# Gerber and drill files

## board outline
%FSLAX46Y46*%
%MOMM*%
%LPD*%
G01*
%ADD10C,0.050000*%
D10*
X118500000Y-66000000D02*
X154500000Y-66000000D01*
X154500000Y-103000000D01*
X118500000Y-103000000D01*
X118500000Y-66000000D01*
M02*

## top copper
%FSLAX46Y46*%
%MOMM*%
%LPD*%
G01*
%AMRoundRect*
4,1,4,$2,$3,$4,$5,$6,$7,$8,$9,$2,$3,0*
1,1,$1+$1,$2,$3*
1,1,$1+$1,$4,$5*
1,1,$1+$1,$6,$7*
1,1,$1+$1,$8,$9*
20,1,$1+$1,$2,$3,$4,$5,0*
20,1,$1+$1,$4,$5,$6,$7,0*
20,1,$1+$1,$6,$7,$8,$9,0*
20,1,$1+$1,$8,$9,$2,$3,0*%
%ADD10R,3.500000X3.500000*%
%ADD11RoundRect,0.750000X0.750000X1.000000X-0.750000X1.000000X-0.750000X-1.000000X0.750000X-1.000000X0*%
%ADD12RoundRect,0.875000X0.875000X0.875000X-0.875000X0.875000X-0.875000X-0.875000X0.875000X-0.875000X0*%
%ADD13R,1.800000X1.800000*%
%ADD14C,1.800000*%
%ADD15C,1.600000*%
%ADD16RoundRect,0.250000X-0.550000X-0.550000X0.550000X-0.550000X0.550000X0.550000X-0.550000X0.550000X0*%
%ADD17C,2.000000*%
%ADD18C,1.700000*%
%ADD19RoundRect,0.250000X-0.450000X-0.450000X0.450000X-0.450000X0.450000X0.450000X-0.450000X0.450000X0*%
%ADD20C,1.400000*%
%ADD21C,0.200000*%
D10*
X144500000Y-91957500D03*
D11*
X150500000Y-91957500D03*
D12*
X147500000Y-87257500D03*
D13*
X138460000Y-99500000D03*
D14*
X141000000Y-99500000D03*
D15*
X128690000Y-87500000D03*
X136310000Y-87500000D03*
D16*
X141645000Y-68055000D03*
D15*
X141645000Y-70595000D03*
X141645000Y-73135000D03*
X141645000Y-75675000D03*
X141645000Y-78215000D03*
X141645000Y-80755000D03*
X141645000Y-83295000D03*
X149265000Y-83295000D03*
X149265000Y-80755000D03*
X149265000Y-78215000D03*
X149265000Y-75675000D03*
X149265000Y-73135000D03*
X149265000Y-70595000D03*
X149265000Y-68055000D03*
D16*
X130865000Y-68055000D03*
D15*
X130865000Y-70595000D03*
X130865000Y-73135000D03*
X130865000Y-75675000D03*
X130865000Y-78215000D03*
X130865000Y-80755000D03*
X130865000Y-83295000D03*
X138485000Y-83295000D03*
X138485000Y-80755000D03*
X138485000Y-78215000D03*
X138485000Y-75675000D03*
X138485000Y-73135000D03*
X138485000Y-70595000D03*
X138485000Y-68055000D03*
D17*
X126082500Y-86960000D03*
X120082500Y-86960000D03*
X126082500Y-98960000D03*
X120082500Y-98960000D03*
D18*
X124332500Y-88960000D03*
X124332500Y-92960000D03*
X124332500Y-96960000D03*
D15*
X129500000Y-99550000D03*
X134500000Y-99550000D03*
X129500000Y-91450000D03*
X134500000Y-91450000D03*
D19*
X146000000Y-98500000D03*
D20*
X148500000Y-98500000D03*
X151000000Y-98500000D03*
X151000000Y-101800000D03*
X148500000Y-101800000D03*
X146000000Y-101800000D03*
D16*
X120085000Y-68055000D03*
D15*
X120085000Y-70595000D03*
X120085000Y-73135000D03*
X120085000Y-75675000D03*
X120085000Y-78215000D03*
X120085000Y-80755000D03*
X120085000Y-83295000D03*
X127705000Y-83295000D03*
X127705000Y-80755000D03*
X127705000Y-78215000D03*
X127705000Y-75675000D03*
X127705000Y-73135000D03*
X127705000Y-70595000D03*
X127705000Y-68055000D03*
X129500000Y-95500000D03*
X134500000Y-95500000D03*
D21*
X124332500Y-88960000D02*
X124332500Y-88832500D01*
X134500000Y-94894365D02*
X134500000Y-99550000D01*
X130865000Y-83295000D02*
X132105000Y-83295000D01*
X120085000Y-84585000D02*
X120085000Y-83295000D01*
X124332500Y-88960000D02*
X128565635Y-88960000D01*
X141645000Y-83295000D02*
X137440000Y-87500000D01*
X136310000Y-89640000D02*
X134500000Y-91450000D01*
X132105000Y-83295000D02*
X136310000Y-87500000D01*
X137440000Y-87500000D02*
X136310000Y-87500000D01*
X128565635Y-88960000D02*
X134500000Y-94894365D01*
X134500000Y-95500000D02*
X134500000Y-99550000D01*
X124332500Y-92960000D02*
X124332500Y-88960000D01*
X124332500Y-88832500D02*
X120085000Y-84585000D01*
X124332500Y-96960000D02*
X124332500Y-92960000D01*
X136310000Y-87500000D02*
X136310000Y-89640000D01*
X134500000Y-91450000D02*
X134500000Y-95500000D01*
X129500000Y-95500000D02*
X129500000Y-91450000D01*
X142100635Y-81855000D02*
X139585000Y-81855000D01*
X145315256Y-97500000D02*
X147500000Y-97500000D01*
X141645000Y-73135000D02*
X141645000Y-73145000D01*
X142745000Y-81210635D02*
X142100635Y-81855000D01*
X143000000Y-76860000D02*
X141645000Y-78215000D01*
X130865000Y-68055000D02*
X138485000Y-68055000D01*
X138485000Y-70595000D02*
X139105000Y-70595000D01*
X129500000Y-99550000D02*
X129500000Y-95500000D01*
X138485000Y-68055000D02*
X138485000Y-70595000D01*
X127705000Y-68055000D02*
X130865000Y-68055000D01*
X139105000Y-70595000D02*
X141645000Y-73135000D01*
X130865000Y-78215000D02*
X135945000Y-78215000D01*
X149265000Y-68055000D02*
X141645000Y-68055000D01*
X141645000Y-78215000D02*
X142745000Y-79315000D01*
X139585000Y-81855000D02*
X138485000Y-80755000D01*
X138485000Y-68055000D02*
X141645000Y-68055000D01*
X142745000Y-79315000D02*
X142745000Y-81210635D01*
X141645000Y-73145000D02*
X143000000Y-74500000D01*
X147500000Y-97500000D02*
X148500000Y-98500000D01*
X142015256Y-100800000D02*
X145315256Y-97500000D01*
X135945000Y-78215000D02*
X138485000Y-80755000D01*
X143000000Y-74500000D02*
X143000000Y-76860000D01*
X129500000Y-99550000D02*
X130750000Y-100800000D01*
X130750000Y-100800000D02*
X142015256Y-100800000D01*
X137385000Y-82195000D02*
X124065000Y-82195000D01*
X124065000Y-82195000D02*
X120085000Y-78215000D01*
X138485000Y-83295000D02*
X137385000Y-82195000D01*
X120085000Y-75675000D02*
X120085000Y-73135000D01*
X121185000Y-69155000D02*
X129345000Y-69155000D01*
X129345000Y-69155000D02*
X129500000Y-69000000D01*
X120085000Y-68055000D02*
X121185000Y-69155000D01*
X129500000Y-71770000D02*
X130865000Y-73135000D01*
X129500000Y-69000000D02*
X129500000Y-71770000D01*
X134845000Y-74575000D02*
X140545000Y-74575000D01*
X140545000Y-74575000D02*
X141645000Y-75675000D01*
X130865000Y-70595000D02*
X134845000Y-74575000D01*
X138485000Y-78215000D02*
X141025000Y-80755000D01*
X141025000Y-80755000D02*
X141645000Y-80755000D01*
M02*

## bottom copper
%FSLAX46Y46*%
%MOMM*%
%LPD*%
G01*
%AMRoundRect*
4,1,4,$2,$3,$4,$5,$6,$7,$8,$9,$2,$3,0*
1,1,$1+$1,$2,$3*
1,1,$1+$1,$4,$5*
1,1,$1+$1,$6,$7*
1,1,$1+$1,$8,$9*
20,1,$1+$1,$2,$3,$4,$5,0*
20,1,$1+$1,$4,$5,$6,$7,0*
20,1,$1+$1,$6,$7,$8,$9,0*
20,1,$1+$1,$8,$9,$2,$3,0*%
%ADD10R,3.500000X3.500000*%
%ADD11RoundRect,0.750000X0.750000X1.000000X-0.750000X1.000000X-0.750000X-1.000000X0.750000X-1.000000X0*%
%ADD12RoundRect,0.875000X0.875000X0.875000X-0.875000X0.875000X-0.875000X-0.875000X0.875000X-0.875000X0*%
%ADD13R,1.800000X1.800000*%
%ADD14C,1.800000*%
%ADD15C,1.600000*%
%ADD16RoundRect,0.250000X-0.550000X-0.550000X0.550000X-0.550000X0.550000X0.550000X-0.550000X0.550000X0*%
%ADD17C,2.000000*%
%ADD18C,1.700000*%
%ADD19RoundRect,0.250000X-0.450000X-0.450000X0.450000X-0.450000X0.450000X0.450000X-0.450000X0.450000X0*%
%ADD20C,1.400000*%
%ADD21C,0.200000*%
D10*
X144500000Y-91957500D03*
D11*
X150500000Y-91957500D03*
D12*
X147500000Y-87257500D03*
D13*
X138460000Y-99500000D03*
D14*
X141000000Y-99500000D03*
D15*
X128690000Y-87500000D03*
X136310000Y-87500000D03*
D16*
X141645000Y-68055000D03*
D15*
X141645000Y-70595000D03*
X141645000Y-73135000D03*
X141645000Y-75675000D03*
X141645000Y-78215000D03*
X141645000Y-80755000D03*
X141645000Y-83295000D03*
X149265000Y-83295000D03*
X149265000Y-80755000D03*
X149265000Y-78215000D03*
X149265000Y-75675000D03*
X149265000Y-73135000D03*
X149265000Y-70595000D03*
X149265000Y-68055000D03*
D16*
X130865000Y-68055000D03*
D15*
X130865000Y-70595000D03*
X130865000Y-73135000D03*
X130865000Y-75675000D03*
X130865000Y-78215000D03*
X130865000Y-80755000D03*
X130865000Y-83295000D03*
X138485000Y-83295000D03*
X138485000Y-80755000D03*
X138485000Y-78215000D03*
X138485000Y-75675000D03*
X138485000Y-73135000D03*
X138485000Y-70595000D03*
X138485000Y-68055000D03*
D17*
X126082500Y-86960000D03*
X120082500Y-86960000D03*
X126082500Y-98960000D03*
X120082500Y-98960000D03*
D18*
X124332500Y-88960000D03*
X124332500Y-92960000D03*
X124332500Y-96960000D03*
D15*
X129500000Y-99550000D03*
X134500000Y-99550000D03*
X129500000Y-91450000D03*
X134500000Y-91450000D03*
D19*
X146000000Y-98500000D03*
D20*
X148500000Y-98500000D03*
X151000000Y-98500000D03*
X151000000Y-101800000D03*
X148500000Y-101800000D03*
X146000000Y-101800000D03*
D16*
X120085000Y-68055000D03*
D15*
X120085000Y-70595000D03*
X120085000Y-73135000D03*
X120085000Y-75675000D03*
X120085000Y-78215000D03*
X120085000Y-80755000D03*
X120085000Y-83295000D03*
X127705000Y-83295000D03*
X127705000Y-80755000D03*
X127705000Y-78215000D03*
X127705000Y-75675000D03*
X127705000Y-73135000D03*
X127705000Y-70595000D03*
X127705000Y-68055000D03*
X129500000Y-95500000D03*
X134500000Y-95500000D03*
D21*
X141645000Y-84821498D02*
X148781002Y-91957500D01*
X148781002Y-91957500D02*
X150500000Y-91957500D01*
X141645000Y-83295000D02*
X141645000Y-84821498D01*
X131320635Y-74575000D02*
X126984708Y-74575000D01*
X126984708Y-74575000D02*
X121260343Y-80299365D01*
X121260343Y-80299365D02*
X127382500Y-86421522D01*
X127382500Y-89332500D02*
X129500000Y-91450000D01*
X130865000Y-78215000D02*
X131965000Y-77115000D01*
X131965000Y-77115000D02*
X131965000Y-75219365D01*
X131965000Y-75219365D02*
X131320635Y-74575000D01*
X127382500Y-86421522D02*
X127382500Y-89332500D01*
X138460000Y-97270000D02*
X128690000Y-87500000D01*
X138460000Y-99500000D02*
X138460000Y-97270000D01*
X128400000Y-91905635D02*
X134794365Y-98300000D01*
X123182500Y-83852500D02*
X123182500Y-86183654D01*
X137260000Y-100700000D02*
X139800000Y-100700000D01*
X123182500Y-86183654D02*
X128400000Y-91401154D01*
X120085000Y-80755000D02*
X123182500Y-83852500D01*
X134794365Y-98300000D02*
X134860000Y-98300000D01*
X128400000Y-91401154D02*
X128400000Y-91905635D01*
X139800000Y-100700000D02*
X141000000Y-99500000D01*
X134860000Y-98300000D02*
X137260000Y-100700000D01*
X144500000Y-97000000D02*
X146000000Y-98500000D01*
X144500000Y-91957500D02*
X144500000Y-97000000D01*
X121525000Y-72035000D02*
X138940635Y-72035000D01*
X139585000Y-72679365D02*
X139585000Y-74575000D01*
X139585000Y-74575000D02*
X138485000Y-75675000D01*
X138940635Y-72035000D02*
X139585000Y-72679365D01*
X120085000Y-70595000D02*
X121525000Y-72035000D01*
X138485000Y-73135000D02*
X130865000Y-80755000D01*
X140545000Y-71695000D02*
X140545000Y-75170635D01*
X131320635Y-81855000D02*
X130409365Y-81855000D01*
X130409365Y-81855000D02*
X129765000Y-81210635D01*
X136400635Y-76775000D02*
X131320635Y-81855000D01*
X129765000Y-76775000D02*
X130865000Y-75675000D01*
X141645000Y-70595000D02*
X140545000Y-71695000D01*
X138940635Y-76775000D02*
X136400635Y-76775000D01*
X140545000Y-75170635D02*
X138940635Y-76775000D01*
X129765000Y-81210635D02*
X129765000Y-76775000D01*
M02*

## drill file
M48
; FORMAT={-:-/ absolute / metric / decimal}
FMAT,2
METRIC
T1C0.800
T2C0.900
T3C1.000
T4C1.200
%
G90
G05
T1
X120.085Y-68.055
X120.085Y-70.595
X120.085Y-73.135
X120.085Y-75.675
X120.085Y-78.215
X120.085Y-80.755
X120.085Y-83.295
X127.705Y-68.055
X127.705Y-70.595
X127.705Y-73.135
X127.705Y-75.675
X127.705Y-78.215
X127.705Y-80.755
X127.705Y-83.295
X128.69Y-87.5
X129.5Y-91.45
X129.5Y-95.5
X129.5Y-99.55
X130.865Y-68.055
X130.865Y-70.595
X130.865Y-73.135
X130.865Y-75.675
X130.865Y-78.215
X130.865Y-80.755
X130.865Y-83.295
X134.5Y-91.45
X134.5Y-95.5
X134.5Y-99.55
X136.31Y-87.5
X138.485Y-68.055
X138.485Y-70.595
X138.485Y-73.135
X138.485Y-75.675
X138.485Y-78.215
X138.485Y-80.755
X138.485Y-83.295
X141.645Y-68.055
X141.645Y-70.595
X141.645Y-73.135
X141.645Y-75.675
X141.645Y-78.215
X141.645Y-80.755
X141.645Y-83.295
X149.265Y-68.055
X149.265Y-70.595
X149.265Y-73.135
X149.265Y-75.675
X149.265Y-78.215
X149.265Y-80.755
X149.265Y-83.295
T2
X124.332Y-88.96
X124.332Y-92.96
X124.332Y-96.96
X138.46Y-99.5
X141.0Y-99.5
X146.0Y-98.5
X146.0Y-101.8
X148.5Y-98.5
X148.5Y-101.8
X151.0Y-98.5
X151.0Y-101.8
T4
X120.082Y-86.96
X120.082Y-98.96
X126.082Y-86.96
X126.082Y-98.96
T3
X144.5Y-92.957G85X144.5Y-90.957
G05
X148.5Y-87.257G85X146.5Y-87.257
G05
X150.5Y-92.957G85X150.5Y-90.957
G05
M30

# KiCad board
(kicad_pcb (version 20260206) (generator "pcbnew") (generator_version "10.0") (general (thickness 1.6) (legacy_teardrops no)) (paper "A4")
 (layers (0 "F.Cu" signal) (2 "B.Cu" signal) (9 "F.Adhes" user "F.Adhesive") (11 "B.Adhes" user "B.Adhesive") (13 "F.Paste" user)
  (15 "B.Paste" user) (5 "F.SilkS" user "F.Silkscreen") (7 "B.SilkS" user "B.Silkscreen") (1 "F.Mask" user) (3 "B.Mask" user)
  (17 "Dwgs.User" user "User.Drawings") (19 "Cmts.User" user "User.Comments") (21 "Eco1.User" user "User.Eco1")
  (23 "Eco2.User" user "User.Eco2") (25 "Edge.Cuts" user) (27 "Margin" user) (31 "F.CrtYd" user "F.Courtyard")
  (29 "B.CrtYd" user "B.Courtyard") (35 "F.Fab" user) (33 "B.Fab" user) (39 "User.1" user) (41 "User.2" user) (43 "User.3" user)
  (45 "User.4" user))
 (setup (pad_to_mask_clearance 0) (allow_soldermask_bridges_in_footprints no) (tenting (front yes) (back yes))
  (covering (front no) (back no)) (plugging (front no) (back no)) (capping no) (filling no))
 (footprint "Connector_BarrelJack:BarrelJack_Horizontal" (layer "F.Cu") (at 144.5 91.9575 180)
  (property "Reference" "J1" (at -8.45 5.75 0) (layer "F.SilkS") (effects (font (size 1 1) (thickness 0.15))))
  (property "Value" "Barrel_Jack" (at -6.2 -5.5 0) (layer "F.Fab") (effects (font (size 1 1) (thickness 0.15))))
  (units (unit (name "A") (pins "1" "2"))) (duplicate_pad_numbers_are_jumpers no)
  (pad "1" thru_hole rect (at 0 0 180) (size 3.5 3.5) (drill oval 1 3) (layers "*.Cu" "*.Mask") (remove_unused_layers no)
   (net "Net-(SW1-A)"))
  (pad "2" thru_hole roundrect (at -6 0 180) (size 3 3.5) (drill oval 1 3) (layers "*.Cu" "*.Mask") (remove_unused_layers no)
   (roundrect_rratio 0.25) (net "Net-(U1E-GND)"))
  (pad "3" thru_hole roundrect (at -3 4.7 180) (size 3.5 3.5) (drill oval 3 1) (layers "*.Cu" "*.Mask") (remove_unused_layers no)
   (roundrect_rratio 0.25)))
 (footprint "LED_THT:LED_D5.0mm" (layer "F.Cu") (at 138.46 99.5)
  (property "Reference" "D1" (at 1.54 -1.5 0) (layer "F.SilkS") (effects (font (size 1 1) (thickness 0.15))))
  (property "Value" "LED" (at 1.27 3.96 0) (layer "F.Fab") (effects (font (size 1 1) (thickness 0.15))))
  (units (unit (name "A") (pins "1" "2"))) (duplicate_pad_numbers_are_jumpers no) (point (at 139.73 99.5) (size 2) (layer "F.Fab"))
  (pad "1" thru_hole rect (at 0 0) (size 1.8 1.8) (drill 0.9) (layers "*.Cu" "*.Mask") (remove_unused_layers no) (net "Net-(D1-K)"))
  (pad "2" thru_hole circle (at 2.54 0) (size 1.8 1.8) (drill 0.9) (layers "*.Cu" "*.Mask") (remove_unused_layers no) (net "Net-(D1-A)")))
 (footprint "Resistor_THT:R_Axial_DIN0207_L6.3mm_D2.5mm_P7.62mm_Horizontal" (layer "F.Cu") (at 128.69 87.5)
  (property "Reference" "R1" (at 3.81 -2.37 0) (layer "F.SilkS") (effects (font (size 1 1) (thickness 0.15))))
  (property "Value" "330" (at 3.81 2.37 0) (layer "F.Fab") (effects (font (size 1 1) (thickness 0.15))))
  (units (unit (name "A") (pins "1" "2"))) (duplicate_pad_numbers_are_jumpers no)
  (pad "1" thru_hole circle (at 0 0) (size 1.6 1.6) (drill 0.8) (layers "*.Cu" "*.Mask") (remove_unused_layers no) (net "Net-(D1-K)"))
  (pad "2" thru_hole circle (at 7.62 0) (size 1.6 1.6) (drill 0.8) (layers "*.Cu" "*.Mask") (remove_unused_layers no) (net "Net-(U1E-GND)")))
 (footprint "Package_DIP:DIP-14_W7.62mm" (layer "F.Cu") (at 141.645 68.055)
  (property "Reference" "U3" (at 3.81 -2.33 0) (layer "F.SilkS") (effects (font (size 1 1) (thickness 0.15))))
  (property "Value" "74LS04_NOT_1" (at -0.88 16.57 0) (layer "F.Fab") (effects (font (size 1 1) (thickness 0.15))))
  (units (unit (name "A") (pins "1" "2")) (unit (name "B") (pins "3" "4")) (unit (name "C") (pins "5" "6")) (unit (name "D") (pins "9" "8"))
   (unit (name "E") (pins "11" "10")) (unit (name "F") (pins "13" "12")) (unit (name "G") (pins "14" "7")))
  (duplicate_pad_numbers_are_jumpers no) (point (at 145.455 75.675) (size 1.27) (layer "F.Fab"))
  (pad "1" thru_hole roundrect (at 0 0) (size 1.6 1.6) (drill 0.8) (layers "*.Cu" "*.Mask") (remove_unused_layers no)
   (roundrect_rratio 0.15625) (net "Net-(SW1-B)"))
  (pad "2" thru_hole circle (at 0 2.54) (size 1.6 1.6) (drill 0.8) (layers "*.Cu" "*.Mask") (remove_unused_layers no) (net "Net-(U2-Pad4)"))
  (pad "3" thru_hole circle (at 0 5.08) (size 1.6 1.6) (drill 0.8) (layers "*.Cu" "*.Mask") (remove_unused_layers no) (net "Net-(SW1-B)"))
  (pad "4" thru_hole circle (at 0 7.62) (size 1.6 1.6) (drill 0.8) (layers "*.Cu" "*.Mask") (remove_unused_layers no) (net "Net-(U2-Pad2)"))
  (pad "5" thru_hole circle (at 0 10.16) (size 1.6 1.6) (drill 0.8) (layers "*.Cu" "*.Mask") (remove_unused_layers no) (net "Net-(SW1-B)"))
  (pad "6" thru_hole circle (at 0 12.7) (size 1.6 1.6) (drill 0.8) (layers "*.Cu" "*.Mask") (remove_unused_layers no) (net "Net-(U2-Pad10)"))
  (pad "7" thru_hole circle (at 0 15.24) (size 1.6 1.6) (drill 0.8) (layers "*.Cu" "*.Mask") (remove_unused_layers no) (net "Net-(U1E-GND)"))
  (pad "8" thru_hole circle (at 7.62 15.24) (size 1.6 1.6) (drill 0.8) (layers "*.Cu" "*.Mask") (remove_unused_layers no)
   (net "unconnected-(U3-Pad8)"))
  (pad "9" thru_hole circle (at 7.62 12.7) (size 1.6 1.6) (drill 0.8) (layers "*.Cu" "*.Mask") (remove_unused_layers no)
   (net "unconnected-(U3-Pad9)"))
  (pad "10" thru_hole circle (at 7.62 10.16) (size 1.6 1.6) (drill 0.8) (layers "*.Cu" "*.Mask") (remove_unused_layers no)
   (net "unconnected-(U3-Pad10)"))
  (pad "11" thru_hole circle (at 7.62 7.62) (size 1.6 1.6) (drill 0.8) (layers "*.Cu" "*.Mask") (remove_unused_layers no)
   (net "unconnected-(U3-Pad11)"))
  (pad "12" thru_hole circle (at 7.62 5.08) (size 1.6 1.6) (drill 0.8) (layers "*.Cu" "*.Mask") (remove_unused_layers no)
   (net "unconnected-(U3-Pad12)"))
  (pad "13" thru_hole circle (at 7.62 2.54) (size 1.6 1.6) (drill 0.8) (layers "*.Cu" "*.Mask") (remove_unused_layers no)
   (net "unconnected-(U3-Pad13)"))
  (pad "14" thru_hole circle (at 7.62 0) (size 1.6 1.6) (drill 0.8) (layers "*.Cu" "*.Mask") (remove_unused_layers no) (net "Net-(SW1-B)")))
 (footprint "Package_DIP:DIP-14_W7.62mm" (layer "F.Cu") (at 130.865 68.055)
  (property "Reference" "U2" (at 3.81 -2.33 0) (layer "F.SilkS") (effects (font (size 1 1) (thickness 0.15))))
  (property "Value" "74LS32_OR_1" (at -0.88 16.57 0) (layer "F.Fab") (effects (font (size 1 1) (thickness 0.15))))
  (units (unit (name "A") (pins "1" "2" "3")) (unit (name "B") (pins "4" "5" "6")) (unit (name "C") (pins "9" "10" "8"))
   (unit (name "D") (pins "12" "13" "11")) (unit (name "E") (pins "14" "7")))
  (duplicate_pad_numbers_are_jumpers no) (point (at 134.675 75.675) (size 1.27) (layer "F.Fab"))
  (pad "1" thru_hole roundrect (at 0 0) (size 1.6 1.6) (drill 0.8) (layers "*.Cu" "*.Mask") (remove_unused_layers no)
   (roundrect_rratio 0.15625) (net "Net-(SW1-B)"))
  (pad "2" thru_hole circle (at 0 2.54) (size 1.6 1.6) (drill 0.8) (layers "*.Cu" "*.Mask") (remove_unused_layers no) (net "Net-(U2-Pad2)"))
  (pad "3" thru_hole circle (at 0 5.08) (size 1.6 1.6) (drill 0.8) (layers "*.Cu" "*.Mask") (remove_unused_layers no) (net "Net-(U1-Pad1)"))
  (pad "4" thru_hole circle (at 0 7.62) (size 1.6 1.6) (drill 0.8) (layers "*.Cu" "*.Mask") (remove_unused_layers no) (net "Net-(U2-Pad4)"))
  (pad "5" thru_hole circle (at 0 10.16) (size 1.6 1.6) (drill 0.8) (layers "*.Cu" "*.Mask") (remove_unused_layers no) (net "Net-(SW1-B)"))
  (pad "6" thru_hole circle (at 0 12.7) (size 1.6 1.6) (drill 0.8) (layers "*.Cu" "*.Mask") (remove_unused_layers no) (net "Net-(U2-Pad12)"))
  (pad "7" thru_hole circle (at 0 15.24) (size 1.6 1.6) (drill 0.8) (layers "*.Cu" "*.Mask") (remove_unused_layers no) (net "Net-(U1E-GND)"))
  (pad "8" thru_hole circle (at 7.62 15.24) (size 1.6 1.6) (drill 0.8) (layers "*.Cu" "*.Mask") (remove_unused_layers no)
   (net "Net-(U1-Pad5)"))
  (pad "9" thru_hole circle (at 7.62 12.7) (size 1.6 1.6) (drill 0.8) (layers "*.Cu" "*.Mask") (remove_unused_layers no) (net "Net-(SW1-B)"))
  (pad "10" thru_hole circle (at 7.62 10.16) (size 1.6 1.6) (drill 0.8) (layers "*.Cu" "*.Mask") (remove_unused_layers no)
   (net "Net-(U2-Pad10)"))
  (pad "11" thru_hole circle (at 7.62 7.62) (size 1.6 1.6) (drill 0.8) (layers "*.Cu" "*.Mask") (remove_unused_layers no)
   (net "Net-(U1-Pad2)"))
  (pad "12" thru_hole circle (at 7.62 5.08) (size 1.6 1.6) (drill 0.8) (layers "*.Cu" "*.Mask") (remove_unused_layers no)
   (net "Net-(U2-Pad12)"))
  (pad "13" thru_hole circle (at 7.62 2.54) (size 1.6 1.6) (drill 0.8) (layers "*.Cu" "*.Mask") (remove_unused_layers no)
   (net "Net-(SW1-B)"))
  (pad "14" thru_hole circle (at 7.62 0) (size 1.6 1.6) (drill 0.8) (layers "*.Cu" "*.Mask") (remove_unused_layers no) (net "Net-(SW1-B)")))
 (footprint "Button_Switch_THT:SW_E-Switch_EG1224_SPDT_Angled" (layer "F.Cu") (at 124.3325 88.96 -90)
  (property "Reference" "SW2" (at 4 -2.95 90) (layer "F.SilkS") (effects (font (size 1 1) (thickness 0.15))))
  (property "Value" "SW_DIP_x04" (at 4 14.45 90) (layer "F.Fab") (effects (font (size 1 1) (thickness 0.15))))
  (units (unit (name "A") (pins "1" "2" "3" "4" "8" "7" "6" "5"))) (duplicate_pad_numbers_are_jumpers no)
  (pad "" thru_hole circle (at -2 -1.75 270) (size 2 2) (drill 1.2) (layers "*.Cu" "*.Mask") (remove_unused_layers no))
  (pad "" thru_hole circle (at -2 4.25 270) (size 2 2) (drill 1.2) (layers "*.Cu" "*.Mask") (remove_unused_layers no))
  (pad "" thru_hole circle (at 10 -1.75 270) (size 2 2) (drill 1.2) (layers "*.Cu" "*.Mask") (remove_unused_layers no))
  (pad "" thru_hole circle (at 10 4.25 270) (size 2 2) (drill 1.2) (layers "*.Cu" "*.Mask") (remove_unused_layers no))
  (pad "1" thru_hole circle (at 0 0 270) (size 1.7 1.7) (drill 0.9) (layers "*.Cu" "*.Mask") (remove_unused_layers no) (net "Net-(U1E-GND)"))
  (pad "2" thru_hole circle (at 4 0 270) (size 1.7 1.7) (drill 0.9) (layers "*.Cu" "*.Mask") (remove_unused_layers no) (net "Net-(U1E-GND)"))
  (pad "3" thru_hole circle (at 8 0 270) (size 1.7 1.7) (drill 0.9) (layers "*.Cu" "*.Mask") (remove_unused_layers no) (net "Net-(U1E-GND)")))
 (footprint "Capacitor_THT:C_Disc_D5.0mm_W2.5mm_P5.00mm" (layer "F.Cu") (at 129.5 99.55)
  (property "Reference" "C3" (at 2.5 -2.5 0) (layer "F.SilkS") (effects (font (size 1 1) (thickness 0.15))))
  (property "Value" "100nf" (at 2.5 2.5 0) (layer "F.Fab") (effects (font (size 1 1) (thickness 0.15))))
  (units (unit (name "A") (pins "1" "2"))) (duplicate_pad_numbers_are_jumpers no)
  (pad "1" thru_hole circle (at 0 0) (size 1.6 1.6) (drill 0.8) (layers "*.Cu" "*.Mask") (remove_unused_layers no) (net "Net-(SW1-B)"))
  (pad "2" thru_hole circle (at 5 0) (size 1.6 1.6) (drill 0.8) (layers "*.Cu" "*.Mask") (remove_unused_layers no) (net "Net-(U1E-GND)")))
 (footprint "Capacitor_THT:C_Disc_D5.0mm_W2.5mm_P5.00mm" (layer "F.Cu") (at 129.5 91.45)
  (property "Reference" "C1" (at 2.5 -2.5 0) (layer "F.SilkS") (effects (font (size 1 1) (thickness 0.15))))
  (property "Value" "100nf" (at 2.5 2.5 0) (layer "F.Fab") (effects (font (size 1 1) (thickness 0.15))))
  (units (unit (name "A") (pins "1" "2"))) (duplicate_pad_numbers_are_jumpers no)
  (pad "1" thru_hole circle (at 0 0) (size 1.6 1.6) (drill 0.8) (layers "*.Cu" "*.Mask") (remove_unused_layers no) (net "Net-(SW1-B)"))
  (pad "2" thru_hole circle (at 5 0) (size 1.6 1.6) (drill 0.8) (layers "*.Cu" "*.Mask") (remove_unused_layers no) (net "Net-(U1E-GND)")))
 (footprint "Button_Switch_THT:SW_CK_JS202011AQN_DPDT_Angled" (layer "F.Cu") (at 146 98.5)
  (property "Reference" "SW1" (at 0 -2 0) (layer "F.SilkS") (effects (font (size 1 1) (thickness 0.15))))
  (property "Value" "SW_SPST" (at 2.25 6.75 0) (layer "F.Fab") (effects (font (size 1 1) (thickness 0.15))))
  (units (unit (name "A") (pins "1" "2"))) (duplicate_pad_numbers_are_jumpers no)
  (pad "1" thru_hole roundrect (at 0 0) (size 1.4 1.4) (drill 0.9) (layers "*.Cu" "*.Mask") (remove_unused_layers no)
   (roundrect_rratio 0.1785714286) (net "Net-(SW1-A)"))
  (pad "2" thru_hole circle (at 2.5 0) (size 1.4 1.4) (drill 0.9) (layers "*.Cu" "*.Mask") (remove_unused_layers no) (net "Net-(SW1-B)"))
  (pad "3" thru_hole circle (at 5 0) (size 1.4 1.4) (drill 0.9) (layers "*.Cu" "*.Mask") (remove_unused_layers no))
  (pad "4" thru_hole circle (at 5 3.3) (size 1.4 1.4) (drill 0.9) (layers "*.Cu" "*.Mask") (remove_unused_layers no))
  (pad "5" thru_hole circle (at 2.5 3.3) (size 1.4 1.4) (drill 0.9) (layers "*.Cu" "*.Mask") (remove_unused_layers no))
  (pad "6" thru_hole circle (at 0 3.3) (size 1.4 1.4) (drill 0.9) (layers "*.Cu" "*.Mask") (remove_unused_layers no)))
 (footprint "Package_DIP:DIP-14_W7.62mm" (layer "F.Cu") (at 120.085 68.055)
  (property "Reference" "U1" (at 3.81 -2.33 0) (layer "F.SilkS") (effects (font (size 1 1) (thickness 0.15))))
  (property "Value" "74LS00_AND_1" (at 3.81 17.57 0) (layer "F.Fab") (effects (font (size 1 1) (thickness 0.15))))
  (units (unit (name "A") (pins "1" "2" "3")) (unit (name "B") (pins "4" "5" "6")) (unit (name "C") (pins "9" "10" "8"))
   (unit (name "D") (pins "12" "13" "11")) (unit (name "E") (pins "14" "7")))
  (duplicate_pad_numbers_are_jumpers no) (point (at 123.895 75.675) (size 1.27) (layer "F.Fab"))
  (pad "1" thru_hole roundrect (at 0 0) (size 1.6 1.6) (drill 0.8) (layers "*.Cu" "*.Mask") (remove_unused_layers no)
   (roundrect_rratio 0.15625) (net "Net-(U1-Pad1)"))
  (pad "2" thru_hole circle (at 0 2.54) (size 1.6 1.6) (drill 0.8) (layers "*.Cu" "*.Mask") (remove_unused_layers no) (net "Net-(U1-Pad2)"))
  (pad "3" thru_hole circle (at 0 5.08) (size 1.6 1.6) (drill 0.8) (layers "*.Cu" "*.Mask") (remove_unused_layers no) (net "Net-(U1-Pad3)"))
  (pad "4" thru_hole circle (at 0 7.62) (size 1.6 1.6) (drill 0.8) (layers "*.Cu" "*.Mask") (remove_unused_layers no) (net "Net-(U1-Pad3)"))
  (pad "5" thru_hole circle (at 0 10.16) (size 1.6 1.6) (drill 0.8) (layers "*.Cu" "*.Mask") (remove_unused_layers no) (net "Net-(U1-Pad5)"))
  (pad "6" thru_hole circle (at 0 12.7) (size 1.6 1.6) (drill 0.8) (layers "*.Cu" "*.Mask") (remove_unused_layers no) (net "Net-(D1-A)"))
  (pad "7" thru_hole circle (at 0 15.24) (size 1.6 1.6) (drill 0.8) (layers "*.Cu" "*.Mask") (remove_unused_layers no) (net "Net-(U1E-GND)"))
  (pad "8" thru_hole circle (at 7.62 15.24) (size 1.6 1.6) (drill 0.8) (layers "*.Cu" "*.Mask") (remove_unused_layers no)
   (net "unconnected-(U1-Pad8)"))
  (pad "9" thru_hole circle (at 7.62 12.7) (size 1.6 1.6) (drill 0.8) (layers "*.Cu" "*.Mask") (remove_unused_layers no)
   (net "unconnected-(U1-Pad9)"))
  (pad "10" thru_hole circle (at 7.62 10.16) (size 1.6 1.6) (drill 0.8) (layers "*.Cu" "*.Mask") (remove_unused_layers no)
   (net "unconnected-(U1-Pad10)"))
  (pad "11" thru_hole circle (at 7.62 7.62) (size 1.6 1.6) (drill 0.8) (layers "*.Cu" "*.Mask") (remove_unused_layers no)
   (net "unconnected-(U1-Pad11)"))
  (pad "12" thru_hole circle (at 7.62 5.08) (size 1.6 1.6) (drill 0.8) (layers "*.Cu" "*.Mask") (remove_unused_layers no)
   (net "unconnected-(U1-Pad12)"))
  (pad "13" thru_hole circle (at 7.62 2.54) (size 1.6 1.6) (drill 0.8) (layers "*.Cu" "*.Mask") (remove_unused_layers no)
   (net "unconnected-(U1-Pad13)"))
  (pad "14" thru_hole circle (at 7.62 0) (size 1.6 1.6) (drill 0.8) (layers "*.Cu" "*.Mask") (remove_unused_layers no) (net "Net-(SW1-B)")))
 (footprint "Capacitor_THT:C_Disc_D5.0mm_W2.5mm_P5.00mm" (layer "F.Cu") (at 129.5 95.5)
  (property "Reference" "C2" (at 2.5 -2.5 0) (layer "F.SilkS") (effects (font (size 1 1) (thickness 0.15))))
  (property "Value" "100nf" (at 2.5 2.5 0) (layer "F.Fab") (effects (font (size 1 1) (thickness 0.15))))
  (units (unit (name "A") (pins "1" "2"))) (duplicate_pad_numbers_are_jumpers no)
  (pad "1" thru_hole circle (at 0 0) (size 1.6 1.6) (drill 0.8) (layers "*.Cu" "*.Mask") (remove_unused_layers no) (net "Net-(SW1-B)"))
  (pad "2" thru_hole circle (at 5 0) (size 1.6 1.6) (drill 0.8) (layers "*.Cu" "*.Mask") (remove_unused_layers no) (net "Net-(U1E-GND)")))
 (gr_rect (start 118.5 66) (end 154.5 103) (stroke (width 0.05) (type default)) (fill no) (layer "Edge.Cuts"))
 (segment (start 124.3325 88.96) (end 124.3325 88.8325) (width 0.2) (layer "F.Cu") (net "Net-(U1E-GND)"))
 (segment (start 134.5 94.894365) (end 134.5 99.55) (width 0.2) (layer "F.Cu") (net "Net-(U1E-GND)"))
 (segment (start 130.865 83.295) (end 132.105 83.295) (width 0.2) (layer "F.Cu") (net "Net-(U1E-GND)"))
 (segment (start 120.085 84.585) (end 120.085 83.295) (width 0.2) (layer "F.Cu") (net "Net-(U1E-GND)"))
 (segment (start 124.3325 88.96) (end 128.565635 88.96) (width 0.2) (layer "F.Cu") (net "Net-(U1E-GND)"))
 (segment (start 141.645 83.295) (end 137.44 87.5) (width 0.2) (layer "F.Cu") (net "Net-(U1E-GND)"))
 (segment (start 136.31 89.64) (end 134.5 91.45) (width 0.2) (layer "F.Cu") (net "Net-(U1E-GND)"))
 (segment (start 132.105 83.295) (end 136.31 87.5) (width 0.2) (layer "F.Cu") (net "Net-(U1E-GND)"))
 (segment (start 137.44 87.5) (end 136.31 87.5) (width 0.2) (layer "F.Cu") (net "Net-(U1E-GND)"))
 (segment (start 128.565635 88.96) (end 134.5 94.894365) (width 0.2) (layer "F.Cu") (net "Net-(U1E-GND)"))
 (segment (start 134.5 95.5) (end 134.5 99.55) (width 0.2) (layer "F.Cu") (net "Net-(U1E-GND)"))
 (segment (start 124.3325 92.96) (end 124.3325 88.96) (width 0.2) (layer "F.Cu") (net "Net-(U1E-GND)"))
 (segment (start 124.3325 88.8325) (end 120.085 84.585) (width 0.2) (layer "F.Cu") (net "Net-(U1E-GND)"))
 (segment (start 124.3325 96.96) (end 124.3325 92.96) (width 0.2) (layer "F.Cu") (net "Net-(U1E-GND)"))
 (segment (start 136.31 87.5) (end 136.31 89.64) (width 0.2) (layer "F.Cu") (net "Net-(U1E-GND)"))
 (segment (start 134.5 91.45) (end 134.5 95.5) (width 0.2) (layer "F.Cu") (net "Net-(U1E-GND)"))
 (segment (start 141.645 84.821498) (end 148.781002 91.9575) (width 0.2) (layer "B.Cu") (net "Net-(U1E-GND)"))
 (segment (start 148.781002 91.9575) (end 150.5 91.9575) (width 0.2) (layer "B.Cu") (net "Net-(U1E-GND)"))
 (segment (start 141.645 83.295) (end 141.645 84.821498) (width 0.2) (layer "B.Cu") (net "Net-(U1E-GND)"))
 (segment (start 129.5 95.5) (end 129.5 91.45) (width 0.2) (layer "F.Cu") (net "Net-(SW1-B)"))
 (segment (start 142.100635 81.855) (end 139.585 81.855) (width 0.2) (layer "F.Cu") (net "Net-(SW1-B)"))
 (segment (start 145.315256 97.5) (end 147.5 97.5) (width 0.2) (layer "F.Cu") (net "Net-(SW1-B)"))
 (segment (start 141.645 73.135) (end 141.645 73.145) (width 0.2) (layer "F.Cu") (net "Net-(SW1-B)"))
 (segment (start 142.745 81.210635) (end 142.100635 81.855) (width 0.2) (layer "F.Cu") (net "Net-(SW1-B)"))
 (segment (start 143 76.86) (end 141.645 78.215) (width 0.2) (layer "F.Cu") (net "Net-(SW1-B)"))
 (segment (start 130.865 68.055) (end 138.485 68.055) (width 0.2) (layer "F.Cu") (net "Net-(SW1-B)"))
 (segment (start 138.485 70.595) (end 139.105 70.595) (width 0.2) (layer "F.Cu") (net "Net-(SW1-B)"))
 (segment (start 129.5 99.55) (end 129.5 95.5) (width 0.2) (layer "F.Cu") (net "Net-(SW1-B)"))
 (segment (start 138.485 68.055) (end 138.485 70.595) (width 0.2) (layer "F.Cu") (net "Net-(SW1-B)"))
 (segment (start 127.705 68.055) (end 130.865 68.055) (width 0.2) (layer "F.Cu") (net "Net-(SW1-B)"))
 (segment (start 139.105 70.595) (end 141.645 73.135) (width 0.2) (layer "F.Cu") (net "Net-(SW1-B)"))
 (segment (start 130.865 78.215) (end 135.945 78.215) (width 0.2) (layer "F.Cu") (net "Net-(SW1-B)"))
 (segment (start 149.265 68.055) (end 141.645 68.055) (width 0.2) (layer "F.Cu") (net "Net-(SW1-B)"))
 (segment (start 141.645 78.215) (end 142.745 79.315) (width 0.2) (layer "F.Cu") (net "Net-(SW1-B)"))
 (segment (start 139.585 81.855) (end 138.485 80.755) (width 0.2) (layer "F.Cu") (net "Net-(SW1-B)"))
 (segment (start 138.485 68.055) (end 141.645 68.055) (width 0.2) (layer "F.Cu") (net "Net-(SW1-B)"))
 (segment (start 142.745 79.315) (end 142.745 81.210635) (width 0.2) (layer "F.Cu") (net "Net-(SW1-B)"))
 (segment (start 141.645 73.145) (end 143 74.5) (width 0.2) (layer "F.Cu") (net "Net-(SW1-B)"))
 (segment (start 147.5 97.5) (end 148.5 98.5) (width 0.2) (layer "F.Cu") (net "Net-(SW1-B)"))
 (segment (start 142.015256 100.8) (end 145.315256 97.5) (width 0.2) (layer "F.Cu") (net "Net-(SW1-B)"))
 (segment (start 135.945 78.215) (end 138.485 80.755) (width 0.2) (layer "F.Cu") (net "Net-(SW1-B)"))
 (segment (start 143 74.5) (end 143 76.86) (width 0.2) (layer "F.Cu") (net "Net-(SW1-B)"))
 (segment (start 129.5 99.55) (end 130.75 100.8) (width 0.2) (layer "F.Cu") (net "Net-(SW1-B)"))
 (segment (start 130.75 100.8) (end 142.015256 100.8) (width 0.2) (layer "F.Cu") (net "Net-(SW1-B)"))
 (segment (start 131.320635 74.575) (end 126.984708 74.575) (width 0.2) (layer "B.Cu") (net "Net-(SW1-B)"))
 (segment (start 126.984708 74.575) (end 121.260343 80.299365) (width 0.2) (layer "B.Cu") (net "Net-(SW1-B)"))
 (segment (start 121.260343 80.299365) (end 127.3825 86.421522) (width 0.2) (layer "B.Cu") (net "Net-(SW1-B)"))
 (segment (start 127.3825 89.3325) (end 129.5 91.45) (width 0.2) (layer "B.Cu") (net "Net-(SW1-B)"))
 (segment (start 130.865 78.215) (end 131.965 77.115) (width 0.2) (layer "B.Cu") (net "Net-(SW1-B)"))
 (segment (start 131.965 77.115) (end 131.965 75.219365) (width 0.2) (layer "B.Cu") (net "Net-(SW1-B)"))
 (segment (start 131.965 75.219365) (end 131.320635 74.575) (width 0.2) (layer "B.Cu") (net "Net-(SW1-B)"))
 (segment (start 127.3825 86.421522) (end 127.3825 89.3325) (width 0.2) (layer "B.Cu") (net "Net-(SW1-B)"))
 (segment (start 138.46 97.27) (end 128.69 87.5) (width 0.2) (layer "B.Cu") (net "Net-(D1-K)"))
 (segment (start 138.46 99.5) (end 138.46 97.27) (width 0.2) (layer "B.Cu") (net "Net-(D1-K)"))
 (segment (start 128.4 91.905635) (end 134.794365 98.3) (width 0.2) (layer "B.Cu") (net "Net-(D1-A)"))
 (segment (start 123.1825 83.8525) (end 123.1825 86.183654) (width 0.2) (layer "B.Cu") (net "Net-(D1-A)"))
 (segment (start 137.26 100.7) (end 139.8 100.7) (width 0.2) (layer "B.Cu") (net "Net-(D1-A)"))
 (segment (start 123.1825 86.183654) (end 128.4 91.401154) (width 0.2) (layer "B.Cu") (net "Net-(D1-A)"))
 (segment (start 120.085 80.755) (end 123.1825 83.8525) (width 0.2) (layer "B.Cu") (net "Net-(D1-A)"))
 (segment (start 134.794365 98.3) (end 134.86 98.3) (width 0.2) (layer "B.Cu") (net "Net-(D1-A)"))
 (segment (start 128.4 91.401154) (end 128.4 91.905635) (width 0.2) (layer "B.Cu") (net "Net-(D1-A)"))
 (segment (start 139.8 100.7) (end 141 99.5) (width 0.2) (layer "B.Cu") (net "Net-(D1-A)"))
 (segment (start 134.86 98.3) (end 137.26 100.7) (width 0.2) (layer "B.Cu") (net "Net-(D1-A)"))
 (segment (start 144.5 97) (end 146 98.5) (width 0.2) (layer "B.Cu") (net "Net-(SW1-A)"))
 (segment (start 144.5 91.9575) (end 144.5 97) (width 0.2) (layer "B.Cu") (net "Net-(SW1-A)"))
 (segment (start 137.385 82.195) (end 124.065 82.195) (width 0.2) (layer "F.Cu") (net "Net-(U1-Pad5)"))
 (segment (start 124.065 82.195) (end 120.085 78.215) (width 0.2) (layer "F.Cu") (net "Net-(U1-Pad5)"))
 (segment (start 138.485 83.295) (end 137.385 82.195) (width 0.2) (layer "F.Cu") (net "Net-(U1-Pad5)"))
 (segment (start 120.085 75.675) (end 120.085 73.135) (width 0.2) (layer "F.Cu") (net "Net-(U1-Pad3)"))
 (segment (start 121.525 72.035) (end 138.940635 72.035) (width 0.2) (layer "B.Cu") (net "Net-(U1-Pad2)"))
 (segment (start 139.585 72.679365) (end 139.585 74.575) (width 0.2) (layer "B.Cu") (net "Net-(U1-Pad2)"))
 (segment (start 139.585 74.575) (end 138.485 75.675) (width 0.2) (layer "B.Cu") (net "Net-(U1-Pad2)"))
 (segment (start 138.940635 72.035) (end 139.585 72.679365) (width 0.2) (layer "B.Cu") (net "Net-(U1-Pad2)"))
 (segment (start 120.085 70.595) (end 121.525 72.035) (width 0.2) (layer "B.Cu") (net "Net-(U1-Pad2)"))
 (segment (start 121.185 69.155) (end 129.345 69.155) (width 0.2) (layer "F.Cu") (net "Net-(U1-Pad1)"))
 (segment (start 129.345 69.155) (end 129.5 69) (width 0.2) (layer "F.Cu") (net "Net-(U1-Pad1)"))
 (segment (start 120.085 68.055) (end 121.185 69.155) (width 0.2) (layer "F.Cu") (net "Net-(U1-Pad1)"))
 (segment (start 129.5 71.77) (end 130.865 73.135) (width 0.2) (layer "F.Cu") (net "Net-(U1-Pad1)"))
 (segment (start 129.5 69) (end 129.5 71.77) (width 0.2) (layer "F.Cu") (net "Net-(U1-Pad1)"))
 (segment (start 138.485 73.135) (end 130.865 80.755) (width 0.2) (layer "B.Cu") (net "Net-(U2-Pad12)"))
 (segment (start 134.845 74.575) (end 140.545 74.575) (width 0.2) (layer "F.Cu") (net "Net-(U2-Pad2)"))
 (segment (start 140.545 74.575) (end 141.645 75.675) (width 0.2) (layer "F.Cu") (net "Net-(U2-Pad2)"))
 (segment (start 130.865 70.595) (end 134.845 74.575) (width 0.2) (layer "F.Cu") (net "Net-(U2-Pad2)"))
 (segment (start 140.545 71.695) (end 140.545 75.170635) (width 0.2) (layer "B.Cu") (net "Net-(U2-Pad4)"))
 (segment (start 131.320635 81.855) (end 130.409365 81.855) (width 0.2) (layer "B.Cu") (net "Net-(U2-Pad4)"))
 (segment (start 130.409365 81.855) (end 129.765 81.210635) (width 0.2) (layer "B.Cu") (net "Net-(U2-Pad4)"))
 (segment (start 136.400635 76.775) (end 131.320635 81.855) (width 0.2) (layer "B.Cu") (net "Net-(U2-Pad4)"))
 (segment (start 129.765 76.775) (end 130.865 75.675) (width 0.2) (layer "B.Cu") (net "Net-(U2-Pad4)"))
 (segment (start 141.645 70.595) (end 140.545 71.695) (width 0.2) (layer "B.Cu") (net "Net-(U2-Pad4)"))
 (segment (start 138.940635 76.775) (end 136.400635 76.775) (width 0.2) (layer "B.Cu") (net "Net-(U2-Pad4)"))
 (segment (start 140.545 75.170635) (end 138.940635 76.775) (width 0.2) (layer "B.Cu") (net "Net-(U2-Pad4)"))
 (segment (start 129.765 81.210635) (end 129.765 76.775) (width 0.2) (layer "B.Cu") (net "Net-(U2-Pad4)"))
 (segment (start 138.485 78.215) (end 141.025 80.755) (width 0.2) (layer "F.Cu") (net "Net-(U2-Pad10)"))
 (segment (start 141.025 80.755) (end 141.645 80.755) (width 0.2) (layer "F.Cu") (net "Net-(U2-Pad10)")))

